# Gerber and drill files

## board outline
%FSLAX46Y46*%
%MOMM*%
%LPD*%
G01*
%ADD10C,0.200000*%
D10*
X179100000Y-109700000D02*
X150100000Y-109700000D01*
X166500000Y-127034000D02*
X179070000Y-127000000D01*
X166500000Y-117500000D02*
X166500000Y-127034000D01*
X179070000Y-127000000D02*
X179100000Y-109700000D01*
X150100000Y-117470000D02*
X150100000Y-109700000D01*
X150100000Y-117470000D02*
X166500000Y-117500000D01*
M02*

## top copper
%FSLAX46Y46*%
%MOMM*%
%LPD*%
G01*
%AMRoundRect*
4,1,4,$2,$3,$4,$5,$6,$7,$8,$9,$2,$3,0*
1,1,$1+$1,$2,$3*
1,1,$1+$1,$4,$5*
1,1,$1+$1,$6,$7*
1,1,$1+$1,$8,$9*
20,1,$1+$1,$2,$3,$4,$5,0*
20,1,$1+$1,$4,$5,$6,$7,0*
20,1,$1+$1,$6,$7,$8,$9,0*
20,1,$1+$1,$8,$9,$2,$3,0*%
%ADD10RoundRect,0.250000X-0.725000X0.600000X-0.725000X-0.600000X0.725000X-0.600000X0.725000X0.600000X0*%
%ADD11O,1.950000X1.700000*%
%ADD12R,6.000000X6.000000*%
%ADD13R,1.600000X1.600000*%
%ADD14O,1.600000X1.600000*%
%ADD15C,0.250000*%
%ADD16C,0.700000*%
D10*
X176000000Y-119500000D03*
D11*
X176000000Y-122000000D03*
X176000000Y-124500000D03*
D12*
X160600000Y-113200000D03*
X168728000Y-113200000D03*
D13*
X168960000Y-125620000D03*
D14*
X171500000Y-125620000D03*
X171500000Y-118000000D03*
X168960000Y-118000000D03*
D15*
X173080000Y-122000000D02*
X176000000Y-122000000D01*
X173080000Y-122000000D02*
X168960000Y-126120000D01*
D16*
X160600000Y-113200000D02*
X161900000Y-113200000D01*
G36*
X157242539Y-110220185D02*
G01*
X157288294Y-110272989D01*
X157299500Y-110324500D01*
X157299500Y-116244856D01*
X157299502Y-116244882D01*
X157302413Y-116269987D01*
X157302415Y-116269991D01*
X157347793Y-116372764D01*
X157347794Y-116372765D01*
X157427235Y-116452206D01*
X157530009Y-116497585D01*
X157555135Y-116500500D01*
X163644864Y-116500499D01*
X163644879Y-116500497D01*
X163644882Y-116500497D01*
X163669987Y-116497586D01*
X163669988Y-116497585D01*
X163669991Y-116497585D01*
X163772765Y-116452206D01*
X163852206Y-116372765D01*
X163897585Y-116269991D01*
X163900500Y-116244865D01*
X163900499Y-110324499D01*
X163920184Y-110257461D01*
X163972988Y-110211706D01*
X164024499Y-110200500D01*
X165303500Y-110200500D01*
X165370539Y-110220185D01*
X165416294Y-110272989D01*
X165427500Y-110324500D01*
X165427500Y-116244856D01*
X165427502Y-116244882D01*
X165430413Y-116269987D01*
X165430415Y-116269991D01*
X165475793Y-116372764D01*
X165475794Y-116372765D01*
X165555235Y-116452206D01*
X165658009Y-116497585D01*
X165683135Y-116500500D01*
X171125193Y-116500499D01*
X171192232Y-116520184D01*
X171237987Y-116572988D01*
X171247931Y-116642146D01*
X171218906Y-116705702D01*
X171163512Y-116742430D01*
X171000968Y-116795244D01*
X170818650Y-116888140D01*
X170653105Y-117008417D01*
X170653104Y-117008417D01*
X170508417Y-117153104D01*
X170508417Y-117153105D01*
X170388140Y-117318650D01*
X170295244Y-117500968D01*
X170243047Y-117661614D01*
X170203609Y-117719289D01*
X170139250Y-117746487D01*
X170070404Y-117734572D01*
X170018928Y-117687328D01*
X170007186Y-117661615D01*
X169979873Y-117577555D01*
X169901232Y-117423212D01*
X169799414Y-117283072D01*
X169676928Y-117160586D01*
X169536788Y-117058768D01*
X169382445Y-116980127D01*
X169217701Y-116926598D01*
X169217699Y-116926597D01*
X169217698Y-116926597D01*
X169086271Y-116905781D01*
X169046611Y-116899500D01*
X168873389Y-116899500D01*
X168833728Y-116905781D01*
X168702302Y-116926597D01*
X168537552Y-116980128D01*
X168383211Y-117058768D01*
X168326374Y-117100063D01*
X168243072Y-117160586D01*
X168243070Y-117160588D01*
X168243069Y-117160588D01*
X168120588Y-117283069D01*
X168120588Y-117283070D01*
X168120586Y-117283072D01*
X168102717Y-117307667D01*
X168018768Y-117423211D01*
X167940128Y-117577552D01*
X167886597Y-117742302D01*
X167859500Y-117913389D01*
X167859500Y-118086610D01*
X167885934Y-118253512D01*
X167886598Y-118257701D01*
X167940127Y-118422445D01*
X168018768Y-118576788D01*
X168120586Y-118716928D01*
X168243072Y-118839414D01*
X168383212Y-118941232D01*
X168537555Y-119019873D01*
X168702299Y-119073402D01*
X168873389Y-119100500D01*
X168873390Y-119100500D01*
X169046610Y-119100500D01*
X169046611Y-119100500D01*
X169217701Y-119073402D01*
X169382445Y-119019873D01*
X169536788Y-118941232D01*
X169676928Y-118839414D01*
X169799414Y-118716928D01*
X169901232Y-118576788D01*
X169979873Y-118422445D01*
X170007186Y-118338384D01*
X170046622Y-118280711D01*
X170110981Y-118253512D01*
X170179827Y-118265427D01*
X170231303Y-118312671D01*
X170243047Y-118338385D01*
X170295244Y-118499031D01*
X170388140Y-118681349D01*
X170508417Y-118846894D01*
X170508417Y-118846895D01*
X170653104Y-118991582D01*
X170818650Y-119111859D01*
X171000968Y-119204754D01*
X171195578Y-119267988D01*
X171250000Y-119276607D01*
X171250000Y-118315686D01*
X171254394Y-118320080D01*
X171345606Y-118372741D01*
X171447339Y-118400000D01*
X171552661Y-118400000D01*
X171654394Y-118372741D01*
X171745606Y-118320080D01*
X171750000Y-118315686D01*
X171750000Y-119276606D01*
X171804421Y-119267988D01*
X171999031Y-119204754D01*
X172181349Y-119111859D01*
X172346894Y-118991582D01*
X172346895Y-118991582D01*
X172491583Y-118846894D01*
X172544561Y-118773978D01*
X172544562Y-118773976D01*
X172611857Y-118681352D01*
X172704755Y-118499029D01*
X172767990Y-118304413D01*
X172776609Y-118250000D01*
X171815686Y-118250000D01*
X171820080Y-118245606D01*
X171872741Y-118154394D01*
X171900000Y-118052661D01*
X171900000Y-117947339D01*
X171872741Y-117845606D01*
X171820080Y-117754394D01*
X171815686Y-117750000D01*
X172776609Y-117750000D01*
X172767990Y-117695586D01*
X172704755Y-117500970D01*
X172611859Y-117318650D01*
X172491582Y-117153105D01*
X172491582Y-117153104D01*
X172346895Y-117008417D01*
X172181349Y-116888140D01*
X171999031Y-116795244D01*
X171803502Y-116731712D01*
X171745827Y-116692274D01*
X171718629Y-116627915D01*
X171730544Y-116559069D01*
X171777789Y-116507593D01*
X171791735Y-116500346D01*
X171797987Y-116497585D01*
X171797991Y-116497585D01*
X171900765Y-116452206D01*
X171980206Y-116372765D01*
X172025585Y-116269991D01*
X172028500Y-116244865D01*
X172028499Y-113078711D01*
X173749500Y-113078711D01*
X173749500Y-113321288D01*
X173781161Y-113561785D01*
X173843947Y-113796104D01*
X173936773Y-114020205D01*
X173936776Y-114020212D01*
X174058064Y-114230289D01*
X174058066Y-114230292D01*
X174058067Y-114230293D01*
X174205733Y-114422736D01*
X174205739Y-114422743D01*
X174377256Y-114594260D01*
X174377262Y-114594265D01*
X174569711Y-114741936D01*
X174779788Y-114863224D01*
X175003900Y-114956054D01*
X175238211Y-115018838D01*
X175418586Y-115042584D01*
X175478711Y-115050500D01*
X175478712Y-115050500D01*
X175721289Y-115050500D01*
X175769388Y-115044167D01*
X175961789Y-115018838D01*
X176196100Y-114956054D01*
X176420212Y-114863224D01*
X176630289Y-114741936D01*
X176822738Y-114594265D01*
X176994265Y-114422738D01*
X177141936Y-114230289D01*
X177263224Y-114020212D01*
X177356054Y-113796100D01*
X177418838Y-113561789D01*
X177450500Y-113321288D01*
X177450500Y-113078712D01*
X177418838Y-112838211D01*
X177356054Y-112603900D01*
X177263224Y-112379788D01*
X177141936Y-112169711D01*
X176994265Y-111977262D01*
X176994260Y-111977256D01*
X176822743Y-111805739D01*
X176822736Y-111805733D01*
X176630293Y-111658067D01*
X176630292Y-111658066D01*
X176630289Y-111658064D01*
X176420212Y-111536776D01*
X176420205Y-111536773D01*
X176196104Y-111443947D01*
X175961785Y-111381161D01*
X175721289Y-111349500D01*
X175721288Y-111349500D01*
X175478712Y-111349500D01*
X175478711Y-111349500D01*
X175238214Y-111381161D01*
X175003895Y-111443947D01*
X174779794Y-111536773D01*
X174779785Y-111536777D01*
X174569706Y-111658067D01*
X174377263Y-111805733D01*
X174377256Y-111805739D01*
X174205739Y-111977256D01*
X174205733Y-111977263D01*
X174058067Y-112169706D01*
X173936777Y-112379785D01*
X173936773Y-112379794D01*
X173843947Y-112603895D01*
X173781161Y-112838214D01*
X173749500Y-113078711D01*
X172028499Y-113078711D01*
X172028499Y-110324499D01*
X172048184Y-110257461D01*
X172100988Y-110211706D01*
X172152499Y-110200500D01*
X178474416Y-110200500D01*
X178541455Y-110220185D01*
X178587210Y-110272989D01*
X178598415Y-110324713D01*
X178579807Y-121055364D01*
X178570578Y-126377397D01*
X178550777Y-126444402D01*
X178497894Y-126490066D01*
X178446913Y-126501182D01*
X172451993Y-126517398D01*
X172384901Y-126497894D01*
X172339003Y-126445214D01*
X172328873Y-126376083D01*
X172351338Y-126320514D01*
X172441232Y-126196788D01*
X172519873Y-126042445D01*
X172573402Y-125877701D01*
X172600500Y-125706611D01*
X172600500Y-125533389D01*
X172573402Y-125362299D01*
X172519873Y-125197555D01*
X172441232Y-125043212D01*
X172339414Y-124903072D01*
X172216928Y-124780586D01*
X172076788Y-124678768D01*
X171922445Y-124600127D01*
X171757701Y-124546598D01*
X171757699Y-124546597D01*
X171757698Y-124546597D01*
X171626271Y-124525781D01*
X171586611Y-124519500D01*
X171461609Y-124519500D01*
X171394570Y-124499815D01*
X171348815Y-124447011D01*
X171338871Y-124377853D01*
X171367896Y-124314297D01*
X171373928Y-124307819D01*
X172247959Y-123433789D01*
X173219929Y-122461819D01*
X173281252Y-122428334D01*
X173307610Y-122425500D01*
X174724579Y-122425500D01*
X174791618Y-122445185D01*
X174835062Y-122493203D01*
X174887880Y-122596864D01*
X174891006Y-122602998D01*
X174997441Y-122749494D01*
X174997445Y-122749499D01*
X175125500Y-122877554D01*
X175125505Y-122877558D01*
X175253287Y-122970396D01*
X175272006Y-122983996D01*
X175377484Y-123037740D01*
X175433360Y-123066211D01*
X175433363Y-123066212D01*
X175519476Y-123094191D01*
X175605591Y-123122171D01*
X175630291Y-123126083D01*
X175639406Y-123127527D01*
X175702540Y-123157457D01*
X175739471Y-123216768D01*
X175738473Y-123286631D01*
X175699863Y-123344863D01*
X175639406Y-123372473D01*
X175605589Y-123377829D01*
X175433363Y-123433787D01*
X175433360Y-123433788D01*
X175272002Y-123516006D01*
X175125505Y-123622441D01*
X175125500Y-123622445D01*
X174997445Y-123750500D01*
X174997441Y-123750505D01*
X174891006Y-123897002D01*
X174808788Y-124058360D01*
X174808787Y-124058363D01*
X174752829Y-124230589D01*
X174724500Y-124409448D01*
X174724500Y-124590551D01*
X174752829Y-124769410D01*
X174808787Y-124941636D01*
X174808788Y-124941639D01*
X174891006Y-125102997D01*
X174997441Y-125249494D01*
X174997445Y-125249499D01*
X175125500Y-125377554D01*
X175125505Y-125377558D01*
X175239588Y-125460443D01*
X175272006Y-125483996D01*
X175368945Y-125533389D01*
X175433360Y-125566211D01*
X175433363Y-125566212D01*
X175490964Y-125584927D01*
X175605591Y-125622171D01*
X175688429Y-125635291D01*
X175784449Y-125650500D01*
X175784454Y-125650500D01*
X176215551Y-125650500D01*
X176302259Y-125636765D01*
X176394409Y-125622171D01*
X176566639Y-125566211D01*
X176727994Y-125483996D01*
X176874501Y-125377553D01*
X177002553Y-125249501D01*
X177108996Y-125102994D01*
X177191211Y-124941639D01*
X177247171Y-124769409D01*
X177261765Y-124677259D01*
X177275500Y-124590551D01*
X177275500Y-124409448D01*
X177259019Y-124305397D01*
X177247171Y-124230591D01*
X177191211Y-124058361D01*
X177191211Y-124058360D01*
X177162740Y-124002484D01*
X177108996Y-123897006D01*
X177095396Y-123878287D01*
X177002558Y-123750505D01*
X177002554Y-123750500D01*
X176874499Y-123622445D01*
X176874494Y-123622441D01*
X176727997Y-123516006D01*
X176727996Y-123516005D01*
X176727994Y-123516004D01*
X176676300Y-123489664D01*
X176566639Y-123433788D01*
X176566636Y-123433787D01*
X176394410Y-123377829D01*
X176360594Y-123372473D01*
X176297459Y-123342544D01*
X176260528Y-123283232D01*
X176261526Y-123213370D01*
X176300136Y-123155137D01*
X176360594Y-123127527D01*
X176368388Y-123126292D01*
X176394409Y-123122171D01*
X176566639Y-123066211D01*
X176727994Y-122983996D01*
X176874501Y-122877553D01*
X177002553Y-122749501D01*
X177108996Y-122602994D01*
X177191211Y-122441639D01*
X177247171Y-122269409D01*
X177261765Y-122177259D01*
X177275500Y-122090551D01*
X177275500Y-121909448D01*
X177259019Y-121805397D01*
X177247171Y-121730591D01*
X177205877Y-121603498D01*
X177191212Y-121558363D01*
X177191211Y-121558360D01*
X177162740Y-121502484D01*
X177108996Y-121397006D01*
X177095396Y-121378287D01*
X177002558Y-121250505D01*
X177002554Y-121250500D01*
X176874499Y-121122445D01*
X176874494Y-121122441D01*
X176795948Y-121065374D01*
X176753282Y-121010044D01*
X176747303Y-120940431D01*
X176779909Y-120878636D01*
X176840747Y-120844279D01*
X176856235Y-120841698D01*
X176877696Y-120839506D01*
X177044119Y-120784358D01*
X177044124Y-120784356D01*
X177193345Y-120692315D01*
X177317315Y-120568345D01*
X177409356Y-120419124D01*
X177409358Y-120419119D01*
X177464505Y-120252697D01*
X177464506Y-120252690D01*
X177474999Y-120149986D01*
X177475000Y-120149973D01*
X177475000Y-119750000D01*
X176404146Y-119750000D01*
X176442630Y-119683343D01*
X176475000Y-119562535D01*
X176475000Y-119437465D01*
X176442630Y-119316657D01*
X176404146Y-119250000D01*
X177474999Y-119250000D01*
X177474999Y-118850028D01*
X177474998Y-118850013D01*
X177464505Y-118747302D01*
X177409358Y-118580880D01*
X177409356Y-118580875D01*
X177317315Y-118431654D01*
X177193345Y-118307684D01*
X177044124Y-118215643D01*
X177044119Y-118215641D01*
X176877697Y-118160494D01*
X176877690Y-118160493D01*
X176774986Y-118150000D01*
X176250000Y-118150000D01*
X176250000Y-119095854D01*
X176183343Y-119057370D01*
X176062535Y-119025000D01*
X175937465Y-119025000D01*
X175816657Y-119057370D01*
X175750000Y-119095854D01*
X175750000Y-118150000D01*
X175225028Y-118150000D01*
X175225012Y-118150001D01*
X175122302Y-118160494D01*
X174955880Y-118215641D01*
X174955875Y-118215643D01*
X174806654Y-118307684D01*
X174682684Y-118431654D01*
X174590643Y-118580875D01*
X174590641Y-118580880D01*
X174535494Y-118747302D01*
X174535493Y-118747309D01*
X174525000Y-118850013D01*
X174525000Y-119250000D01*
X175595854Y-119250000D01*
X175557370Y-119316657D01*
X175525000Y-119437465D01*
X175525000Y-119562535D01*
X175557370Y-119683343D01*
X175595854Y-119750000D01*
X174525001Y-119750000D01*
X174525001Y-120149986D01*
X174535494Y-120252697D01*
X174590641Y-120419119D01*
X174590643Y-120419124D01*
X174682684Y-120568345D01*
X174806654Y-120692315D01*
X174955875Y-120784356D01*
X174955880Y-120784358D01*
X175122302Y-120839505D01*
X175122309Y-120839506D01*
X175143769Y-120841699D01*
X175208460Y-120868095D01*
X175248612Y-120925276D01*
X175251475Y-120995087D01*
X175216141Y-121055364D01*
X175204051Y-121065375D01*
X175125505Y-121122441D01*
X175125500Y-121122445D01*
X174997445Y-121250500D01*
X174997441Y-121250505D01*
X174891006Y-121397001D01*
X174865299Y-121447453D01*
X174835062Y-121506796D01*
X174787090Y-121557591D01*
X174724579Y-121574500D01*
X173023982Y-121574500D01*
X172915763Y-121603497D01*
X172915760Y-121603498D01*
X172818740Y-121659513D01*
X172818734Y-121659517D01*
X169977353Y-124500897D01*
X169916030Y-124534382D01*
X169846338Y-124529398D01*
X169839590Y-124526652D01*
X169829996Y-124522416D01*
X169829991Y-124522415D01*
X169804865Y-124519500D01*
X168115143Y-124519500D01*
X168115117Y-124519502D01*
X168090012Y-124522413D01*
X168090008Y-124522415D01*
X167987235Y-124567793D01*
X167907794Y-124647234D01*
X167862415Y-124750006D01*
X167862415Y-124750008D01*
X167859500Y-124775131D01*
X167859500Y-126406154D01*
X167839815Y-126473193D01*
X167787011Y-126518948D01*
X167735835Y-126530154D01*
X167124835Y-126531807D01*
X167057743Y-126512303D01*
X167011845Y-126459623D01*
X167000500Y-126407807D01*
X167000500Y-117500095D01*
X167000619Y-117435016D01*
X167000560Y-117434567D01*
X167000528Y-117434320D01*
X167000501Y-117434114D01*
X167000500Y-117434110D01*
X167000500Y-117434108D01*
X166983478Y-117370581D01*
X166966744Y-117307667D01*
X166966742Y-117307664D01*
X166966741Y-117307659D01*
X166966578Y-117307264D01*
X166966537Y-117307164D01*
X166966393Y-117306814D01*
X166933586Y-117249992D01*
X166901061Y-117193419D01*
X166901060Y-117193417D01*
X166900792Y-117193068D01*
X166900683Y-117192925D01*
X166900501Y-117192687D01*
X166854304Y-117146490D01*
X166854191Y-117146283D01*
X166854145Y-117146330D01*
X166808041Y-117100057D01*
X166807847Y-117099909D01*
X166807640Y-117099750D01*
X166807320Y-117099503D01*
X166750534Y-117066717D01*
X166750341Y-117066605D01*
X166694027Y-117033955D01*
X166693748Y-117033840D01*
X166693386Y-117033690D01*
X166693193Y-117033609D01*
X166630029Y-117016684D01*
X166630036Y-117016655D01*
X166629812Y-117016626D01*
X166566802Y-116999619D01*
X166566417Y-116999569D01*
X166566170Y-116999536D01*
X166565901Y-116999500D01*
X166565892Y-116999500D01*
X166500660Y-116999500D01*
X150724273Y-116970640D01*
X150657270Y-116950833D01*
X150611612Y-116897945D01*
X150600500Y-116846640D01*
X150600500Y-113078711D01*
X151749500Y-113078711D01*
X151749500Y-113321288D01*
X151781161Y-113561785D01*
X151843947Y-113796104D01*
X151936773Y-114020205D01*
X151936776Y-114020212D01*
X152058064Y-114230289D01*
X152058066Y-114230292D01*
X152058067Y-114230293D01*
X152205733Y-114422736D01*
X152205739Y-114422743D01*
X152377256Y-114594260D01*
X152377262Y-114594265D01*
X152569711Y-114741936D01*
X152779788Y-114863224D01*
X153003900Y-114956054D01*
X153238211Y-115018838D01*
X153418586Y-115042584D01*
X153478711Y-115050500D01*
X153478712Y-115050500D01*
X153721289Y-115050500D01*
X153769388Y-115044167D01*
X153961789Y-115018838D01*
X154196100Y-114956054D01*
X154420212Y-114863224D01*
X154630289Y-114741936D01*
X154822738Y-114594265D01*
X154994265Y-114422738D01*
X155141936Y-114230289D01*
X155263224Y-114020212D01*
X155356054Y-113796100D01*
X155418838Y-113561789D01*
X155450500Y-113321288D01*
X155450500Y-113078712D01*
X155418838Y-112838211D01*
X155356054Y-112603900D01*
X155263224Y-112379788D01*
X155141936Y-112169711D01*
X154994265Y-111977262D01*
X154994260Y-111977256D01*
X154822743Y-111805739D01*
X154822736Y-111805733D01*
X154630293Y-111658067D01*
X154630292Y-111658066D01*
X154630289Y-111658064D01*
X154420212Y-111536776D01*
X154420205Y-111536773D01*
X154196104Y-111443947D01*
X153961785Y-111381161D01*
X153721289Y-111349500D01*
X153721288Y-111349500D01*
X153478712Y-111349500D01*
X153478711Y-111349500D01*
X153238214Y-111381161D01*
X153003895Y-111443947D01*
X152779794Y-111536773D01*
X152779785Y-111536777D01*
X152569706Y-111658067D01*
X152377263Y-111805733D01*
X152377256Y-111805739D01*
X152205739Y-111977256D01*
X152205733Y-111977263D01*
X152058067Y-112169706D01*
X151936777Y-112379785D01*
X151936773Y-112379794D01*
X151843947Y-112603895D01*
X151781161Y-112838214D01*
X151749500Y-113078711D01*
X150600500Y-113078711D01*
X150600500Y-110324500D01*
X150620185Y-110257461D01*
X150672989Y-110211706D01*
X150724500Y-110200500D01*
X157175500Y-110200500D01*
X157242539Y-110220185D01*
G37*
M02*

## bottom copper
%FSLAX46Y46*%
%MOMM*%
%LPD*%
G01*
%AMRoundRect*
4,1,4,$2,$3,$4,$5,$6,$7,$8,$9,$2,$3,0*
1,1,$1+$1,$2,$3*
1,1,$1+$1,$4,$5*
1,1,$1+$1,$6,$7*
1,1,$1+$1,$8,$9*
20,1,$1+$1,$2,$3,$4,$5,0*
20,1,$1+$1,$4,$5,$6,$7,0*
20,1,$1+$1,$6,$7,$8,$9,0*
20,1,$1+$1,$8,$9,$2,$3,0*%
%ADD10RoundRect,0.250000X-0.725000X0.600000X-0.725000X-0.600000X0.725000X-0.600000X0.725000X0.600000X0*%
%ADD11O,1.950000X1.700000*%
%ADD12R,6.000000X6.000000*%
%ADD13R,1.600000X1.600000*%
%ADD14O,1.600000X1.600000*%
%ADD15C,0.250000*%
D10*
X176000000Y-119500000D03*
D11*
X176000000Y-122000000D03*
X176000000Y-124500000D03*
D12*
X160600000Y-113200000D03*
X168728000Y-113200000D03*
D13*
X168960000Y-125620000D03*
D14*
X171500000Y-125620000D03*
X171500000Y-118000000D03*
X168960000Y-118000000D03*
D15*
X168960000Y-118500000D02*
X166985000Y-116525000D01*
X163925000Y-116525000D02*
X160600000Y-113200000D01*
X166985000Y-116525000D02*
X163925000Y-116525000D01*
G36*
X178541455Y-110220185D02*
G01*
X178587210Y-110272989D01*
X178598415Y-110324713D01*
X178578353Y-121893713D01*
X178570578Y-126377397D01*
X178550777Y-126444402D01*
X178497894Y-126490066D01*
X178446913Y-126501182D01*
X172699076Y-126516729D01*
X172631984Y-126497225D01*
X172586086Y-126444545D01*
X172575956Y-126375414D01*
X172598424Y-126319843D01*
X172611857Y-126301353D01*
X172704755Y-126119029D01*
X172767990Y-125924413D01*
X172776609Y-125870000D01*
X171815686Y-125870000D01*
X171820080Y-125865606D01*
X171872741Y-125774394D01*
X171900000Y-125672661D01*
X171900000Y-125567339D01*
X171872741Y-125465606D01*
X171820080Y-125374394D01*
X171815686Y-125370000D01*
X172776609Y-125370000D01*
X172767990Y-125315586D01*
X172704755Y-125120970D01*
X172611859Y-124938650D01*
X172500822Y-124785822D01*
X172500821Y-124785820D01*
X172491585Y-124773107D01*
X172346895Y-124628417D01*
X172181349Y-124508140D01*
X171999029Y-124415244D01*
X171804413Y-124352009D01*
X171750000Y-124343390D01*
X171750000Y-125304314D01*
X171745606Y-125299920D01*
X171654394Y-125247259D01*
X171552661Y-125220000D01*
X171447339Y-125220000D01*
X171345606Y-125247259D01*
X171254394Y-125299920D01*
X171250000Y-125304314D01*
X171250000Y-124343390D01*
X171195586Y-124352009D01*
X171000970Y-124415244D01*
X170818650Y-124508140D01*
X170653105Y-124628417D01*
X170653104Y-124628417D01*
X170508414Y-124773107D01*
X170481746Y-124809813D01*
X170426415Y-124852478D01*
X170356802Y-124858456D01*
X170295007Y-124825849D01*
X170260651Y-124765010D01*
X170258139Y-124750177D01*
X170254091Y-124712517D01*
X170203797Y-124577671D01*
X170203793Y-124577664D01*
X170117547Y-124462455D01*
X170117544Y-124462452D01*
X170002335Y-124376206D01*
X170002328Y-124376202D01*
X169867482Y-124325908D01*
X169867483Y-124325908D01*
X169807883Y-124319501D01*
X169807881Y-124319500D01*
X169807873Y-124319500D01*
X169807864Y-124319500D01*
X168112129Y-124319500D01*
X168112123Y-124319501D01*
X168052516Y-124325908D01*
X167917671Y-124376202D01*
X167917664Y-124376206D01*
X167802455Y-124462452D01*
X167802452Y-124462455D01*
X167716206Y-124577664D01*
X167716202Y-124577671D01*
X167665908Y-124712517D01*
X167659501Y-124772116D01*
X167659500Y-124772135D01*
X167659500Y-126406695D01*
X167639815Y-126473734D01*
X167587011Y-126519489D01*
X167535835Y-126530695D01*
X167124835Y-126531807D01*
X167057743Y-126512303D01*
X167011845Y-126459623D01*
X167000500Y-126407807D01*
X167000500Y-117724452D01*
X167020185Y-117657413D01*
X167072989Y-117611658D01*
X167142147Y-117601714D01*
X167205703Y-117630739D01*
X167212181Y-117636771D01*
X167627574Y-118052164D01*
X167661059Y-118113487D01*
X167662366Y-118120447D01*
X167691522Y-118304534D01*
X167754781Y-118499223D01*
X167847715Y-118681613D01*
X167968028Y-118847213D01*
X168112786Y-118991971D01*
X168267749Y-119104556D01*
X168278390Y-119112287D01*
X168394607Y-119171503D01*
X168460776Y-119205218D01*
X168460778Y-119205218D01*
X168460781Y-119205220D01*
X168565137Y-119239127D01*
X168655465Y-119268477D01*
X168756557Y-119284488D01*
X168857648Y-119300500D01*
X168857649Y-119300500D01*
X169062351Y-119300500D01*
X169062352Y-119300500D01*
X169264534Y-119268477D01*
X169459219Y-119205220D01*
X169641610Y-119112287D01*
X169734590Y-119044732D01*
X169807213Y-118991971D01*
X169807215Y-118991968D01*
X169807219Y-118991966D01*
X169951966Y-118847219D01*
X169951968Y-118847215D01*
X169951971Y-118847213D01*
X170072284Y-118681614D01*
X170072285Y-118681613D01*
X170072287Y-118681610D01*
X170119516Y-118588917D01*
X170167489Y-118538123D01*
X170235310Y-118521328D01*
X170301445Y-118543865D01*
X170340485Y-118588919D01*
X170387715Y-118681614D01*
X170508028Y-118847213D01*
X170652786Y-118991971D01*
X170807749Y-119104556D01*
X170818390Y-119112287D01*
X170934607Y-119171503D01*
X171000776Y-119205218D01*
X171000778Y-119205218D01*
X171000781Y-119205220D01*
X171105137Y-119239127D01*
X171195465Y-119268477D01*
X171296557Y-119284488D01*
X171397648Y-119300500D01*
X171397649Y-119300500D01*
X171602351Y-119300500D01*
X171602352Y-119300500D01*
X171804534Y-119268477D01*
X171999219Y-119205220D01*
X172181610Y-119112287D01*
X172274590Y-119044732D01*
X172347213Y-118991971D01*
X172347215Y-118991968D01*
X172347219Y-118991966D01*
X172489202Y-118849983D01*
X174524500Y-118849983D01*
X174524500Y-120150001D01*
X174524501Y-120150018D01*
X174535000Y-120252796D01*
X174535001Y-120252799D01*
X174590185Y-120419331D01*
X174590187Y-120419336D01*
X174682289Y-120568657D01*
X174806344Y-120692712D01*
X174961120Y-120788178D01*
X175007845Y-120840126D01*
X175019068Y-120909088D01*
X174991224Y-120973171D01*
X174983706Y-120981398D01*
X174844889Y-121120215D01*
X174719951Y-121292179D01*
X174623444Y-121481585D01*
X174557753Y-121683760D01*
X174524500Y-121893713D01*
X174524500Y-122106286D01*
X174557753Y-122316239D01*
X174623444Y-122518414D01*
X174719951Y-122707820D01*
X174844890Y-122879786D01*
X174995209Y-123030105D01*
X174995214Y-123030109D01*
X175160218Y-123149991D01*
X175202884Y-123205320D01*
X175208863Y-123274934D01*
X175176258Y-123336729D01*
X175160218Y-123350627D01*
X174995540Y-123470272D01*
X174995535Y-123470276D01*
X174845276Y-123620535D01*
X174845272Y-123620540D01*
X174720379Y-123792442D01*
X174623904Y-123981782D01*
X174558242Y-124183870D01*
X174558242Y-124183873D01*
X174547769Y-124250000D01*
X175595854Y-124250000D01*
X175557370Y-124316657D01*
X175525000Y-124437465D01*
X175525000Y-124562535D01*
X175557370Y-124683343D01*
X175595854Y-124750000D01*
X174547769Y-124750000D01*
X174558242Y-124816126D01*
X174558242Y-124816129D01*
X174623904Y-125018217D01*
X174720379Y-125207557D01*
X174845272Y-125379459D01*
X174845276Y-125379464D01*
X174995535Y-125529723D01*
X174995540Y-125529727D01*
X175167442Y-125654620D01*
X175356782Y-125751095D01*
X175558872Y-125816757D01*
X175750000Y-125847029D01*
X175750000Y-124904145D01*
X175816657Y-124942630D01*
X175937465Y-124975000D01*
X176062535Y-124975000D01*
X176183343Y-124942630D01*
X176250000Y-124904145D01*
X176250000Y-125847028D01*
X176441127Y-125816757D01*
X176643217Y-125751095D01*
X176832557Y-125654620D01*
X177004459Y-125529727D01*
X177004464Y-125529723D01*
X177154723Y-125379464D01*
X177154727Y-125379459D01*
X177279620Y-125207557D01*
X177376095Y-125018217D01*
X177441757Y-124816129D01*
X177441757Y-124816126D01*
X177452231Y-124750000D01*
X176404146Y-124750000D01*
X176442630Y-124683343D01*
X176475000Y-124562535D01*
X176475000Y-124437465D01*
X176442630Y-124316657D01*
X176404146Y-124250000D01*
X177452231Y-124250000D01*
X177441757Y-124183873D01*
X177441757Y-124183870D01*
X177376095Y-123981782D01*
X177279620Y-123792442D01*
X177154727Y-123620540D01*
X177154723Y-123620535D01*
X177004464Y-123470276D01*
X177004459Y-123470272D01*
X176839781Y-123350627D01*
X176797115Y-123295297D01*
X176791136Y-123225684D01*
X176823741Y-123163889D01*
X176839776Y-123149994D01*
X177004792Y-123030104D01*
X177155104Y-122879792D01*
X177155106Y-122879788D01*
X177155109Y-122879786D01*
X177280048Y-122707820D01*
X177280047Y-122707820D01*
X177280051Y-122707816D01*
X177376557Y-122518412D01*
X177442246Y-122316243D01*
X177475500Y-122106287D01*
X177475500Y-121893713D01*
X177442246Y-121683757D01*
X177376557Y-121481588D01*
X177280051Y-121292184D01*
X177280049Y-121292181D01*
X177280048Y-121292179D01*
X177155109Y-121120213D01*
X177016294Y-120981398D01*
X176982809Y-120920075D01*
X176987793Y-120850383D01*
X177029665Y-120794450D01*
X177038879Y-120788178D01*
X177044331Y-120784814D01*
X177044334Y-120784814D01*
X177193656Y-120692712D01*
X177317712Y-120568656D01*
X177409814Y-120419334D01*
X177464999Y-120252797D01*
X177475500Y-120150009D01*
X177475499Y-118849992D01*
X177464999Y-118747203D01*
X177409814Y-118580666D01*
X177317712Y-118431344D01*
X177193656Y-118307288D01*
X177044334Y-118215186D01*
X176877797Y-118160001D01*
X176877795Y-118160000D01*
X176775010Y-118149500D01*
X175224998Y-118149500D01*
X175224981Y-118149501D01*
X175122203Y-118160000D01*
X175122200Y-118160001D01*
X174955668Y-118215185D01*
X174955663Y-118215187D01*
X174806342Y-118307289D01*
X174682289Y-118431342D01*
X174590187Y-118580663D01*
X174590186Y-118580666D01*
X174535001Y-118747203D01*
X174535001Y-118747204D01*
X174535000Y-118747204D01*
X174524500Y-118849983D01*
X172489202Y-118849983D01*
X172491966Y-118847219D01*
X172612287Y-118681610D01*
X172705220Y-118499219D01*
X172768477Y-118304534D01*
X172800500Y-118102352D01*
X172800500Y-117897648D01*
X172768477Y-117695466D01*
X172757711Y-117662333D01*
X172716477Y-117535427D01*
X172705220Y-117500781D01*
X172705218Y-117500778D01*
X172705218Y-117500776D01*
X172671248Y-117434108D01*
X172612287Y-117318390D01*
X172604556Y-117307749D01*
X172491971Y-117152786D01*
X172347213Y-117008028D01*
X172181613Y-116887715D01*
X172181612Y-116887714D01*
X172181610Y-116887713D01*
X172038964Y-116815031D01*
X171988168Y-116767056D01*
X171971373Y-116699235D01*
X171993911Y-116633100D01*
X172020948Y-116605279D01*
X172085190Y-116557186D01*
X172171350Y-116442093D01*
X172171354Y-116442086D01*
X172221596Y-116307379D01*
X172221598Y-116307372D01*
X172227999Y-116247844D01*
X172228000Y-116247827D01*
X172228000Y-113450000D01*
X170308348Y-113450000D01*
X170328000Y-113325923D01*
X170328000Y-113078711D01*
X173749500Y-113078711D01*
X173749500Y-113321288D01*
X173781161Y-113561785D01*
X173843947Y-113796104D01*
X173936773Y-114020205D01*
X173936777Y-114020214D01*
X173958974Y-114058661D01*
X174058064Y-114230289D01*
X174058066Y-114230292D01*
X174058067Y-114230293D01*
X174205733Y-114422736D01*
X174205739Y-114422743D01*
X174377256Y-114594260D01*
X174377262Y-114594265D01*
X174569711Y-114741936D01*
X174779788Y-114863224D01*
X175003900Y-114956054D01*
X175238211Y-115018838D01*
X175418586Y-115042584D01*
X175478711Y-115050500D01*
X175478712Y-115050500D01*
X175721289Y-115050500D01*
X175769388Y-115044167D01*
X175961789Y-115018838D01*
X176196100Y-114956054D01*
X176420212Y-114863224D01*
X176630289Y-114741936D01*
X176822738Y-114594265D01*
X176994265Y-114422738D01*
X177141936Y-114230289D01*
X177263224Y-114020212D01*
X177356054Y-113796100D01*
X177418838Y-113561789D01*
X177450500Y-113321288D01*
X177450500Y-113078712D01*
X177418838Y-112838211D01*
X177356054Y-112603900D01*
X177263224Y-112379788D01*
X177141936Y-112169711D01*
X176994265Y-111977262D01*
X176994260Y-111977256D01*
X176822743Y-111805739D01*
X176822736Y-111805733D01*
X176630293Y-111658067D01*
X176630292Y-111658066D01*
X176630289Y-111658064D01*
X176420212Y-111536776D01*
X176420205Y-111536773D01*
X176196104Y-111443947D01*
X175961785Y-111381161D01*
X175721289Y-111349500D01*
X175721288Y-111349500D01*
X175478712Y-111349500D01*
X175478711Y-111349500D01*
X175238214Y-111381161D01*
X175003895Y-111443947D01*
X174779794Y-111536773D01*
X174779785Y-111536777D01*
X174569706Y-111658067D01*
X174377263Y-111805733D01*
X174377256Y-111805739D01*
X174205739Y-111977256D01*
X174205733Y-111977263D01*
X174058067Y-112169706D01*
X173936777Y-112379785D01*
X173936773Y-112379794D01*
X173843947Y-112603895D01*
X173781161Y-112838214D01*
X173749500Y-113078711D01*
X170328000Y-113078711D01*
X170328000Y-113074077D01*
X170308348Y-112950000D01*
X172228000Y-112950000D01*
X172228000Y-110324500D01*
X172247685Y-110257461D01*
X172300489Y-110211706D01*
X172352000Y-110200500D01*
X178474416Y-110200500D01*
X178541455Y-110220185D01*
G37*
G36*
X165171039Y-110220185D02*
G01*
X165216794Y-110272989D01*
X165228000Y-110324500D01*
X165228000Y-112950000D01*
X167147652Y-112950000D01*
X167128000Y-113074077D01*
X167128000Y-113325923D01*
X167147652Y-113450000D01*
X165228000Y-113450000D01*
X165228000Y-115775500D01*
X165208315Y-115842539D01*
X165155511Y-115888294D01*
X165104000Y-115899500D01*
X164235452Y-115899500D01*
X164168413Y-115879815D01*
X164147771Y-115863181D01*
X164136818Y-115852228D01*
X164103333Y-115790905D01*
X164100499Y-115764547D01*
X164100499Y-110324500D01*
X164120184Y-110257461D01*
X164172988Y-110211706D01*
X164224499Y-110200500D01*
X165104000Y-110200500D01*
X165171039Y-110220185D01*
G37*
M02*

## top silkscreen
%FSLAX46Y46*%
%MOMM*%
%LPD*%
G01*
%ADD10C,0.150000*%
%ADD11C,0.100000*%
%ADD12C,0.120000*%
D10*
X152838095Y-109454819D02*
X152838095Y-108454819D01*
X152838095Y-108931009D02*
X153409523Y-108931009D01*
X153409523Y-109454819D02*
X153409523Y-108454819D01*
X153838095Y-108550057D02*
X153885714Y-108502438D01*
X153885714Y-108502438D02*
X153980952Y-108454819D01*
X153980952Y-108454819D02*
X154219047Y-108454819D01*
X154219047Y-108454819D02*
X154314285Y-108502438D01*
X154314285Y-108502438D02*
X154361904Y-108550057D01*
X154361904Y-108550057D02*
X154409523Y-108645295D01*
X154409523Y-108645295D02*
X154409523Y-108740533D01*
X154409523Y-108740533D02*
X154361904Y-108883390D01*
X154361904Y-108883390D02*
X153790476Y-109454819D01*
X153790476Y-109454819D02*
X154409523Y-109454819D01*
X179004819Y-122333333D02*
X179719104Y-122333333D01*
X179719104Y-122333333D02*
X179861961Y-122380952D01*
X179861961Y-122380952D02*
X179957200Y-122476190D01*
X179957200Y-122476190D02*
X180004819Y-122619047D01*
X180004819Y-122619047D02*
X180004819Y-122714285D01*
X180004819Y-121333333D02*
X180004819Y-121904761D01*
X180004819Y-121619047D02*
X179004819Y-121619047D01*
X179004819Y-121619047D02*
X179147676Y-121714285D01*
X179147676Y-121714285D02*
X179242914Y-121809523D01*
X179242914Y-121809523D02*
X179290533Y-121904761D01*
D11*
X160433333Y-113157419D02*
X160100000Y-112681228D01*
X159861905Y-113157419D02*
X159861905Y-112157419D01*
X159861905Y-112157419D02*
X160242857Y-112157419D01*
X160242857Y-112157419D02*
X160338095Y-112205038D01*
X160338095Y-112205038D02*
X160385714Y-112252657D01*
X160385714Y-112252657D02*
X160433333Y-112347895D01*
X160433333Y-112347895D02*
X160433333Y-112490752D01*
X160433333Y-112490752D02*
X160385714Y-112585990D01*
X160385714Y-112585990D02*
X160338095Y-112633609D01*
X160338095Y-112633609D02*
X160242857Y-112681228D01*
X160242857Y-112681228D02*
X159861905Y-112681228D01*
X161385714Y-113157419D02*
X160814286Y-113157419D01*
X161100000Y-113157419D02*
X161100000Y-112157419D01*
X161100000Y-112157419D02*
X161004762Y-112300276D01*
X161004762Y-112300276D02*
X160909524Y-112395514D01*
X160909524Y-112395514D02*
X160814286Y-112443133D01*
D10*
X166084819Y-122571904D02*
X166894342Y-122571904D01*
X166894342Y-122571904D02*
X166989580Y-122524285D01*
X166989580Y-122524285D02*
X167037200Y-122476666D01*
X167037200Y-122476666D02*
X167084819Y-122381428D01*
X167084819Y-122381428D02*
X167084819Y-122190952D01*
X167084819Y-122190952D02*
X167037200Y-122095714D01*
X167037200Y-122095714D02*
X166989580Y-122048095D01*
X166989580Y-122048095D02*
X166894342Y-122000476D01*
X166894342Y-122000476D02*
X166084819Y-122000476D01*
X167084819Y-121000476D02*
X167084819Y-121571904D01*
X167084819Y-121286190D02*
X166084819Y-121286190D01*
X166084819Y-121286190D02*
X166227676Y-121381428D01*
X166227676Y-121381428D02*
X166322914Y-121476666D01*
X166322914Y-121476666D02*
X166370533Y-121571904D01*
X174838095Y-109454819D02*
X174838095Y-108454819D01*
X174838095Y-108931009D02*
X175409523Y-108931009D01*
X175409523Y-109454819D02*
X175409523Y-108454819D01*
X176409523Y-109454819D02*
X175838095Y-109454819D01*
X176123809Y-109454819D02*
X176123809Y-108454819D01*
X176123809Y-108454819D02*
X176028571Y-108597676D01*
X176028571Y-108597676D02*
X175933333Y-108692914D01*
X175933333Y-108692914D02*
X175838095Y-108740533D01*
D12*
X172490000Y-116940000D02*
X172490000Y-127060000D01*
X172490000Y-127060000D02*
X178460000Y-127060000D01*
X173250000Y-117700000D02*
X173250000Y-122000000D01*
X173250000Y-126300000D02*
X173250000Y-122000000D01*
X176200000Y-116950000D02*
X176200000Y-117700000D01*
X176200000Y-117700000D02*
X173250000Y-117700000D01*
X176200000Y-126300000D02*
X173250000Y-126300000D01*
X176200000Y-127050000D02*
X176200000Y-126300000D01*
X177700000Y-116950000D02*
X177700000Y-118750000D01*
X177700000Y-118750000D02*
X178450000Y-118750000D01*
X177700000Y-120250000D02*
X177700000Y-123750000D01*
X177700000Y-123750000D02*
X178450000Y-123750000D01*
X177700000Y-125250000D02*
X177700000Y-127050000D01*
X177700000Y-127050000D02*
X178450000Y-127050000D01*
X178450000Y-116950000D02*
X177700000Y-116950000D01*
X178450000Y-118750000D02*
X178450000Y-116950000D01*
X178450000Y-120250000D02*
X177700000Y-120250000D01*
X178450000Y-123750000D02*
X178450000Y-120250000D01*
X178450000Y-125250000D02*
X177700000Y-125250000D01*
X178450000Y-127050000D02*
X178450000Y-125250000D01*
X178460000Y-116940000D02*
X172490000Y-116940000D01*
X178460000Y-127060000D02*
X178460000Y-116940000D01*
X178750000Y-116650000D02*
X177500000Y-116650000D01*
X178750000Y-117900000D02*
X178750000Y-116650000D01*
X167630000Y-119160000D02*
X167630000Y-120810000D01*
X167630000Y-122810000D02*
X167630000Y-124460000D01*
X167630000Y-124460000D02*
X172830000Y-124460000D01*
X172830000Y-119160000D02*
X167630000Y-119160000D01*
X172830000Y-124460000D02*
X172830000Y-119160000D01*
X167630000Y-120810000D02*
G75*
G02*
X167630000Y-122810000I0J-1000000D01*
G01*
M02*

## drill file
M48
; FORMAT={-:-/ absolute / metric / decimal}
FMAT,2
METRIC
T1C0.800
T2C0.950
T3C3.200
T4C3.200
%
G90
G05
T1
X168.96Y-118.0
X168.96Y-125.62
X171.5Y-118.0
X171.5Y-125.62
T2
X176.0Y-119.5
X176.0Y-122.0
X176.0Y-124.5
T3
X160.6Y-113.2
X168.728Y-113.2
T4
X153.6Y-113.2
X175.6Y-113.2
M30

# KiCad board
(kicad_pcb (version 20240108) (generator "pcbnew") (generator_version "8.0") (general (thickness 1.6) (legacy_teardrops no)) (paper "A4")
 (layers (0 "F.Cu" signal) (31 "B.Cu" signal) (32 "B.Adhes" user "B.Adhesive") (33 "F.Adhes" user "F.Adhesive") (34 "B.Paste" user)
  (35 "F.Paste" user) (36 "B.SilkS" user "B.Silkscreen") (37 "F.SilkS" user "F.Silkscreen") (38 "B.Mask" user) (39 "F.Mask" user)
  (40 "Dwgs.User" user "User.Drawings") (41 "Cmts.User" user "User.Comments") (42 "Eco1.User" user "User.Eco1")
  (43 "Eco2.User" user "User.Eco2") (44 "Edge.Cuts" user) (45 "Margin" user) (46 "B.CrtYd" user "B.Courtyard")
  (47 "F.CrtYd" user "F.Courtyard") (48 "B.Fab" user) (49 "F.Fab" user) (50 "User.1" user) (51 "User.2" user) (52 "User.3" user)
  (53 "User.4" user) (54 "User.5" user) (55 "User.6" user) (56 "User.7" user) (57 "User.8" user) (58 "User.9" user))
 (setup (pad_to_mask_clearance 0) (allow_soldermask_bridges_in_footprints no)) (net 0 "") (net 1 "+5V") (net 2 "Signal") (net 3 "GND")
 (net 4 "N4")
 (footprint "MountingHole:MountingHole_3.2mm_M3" (layer "F.Cu") (at 153.6 113.2)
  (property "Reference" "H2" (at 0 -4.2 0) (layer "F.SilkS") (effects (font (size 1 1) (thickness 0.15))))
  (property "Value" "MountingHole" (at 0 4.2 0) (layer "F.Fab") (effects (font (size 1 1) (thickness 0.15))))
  (pad "" np_thru_hole circle (at 0 0) (size 3.2 3.2) (drill 3.2) (layers "*.Cu" "*.Mask")))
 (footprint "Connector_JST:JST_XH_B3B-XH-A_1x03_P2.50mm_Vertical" (layer "F.Cu") (at 176 119.5 -90)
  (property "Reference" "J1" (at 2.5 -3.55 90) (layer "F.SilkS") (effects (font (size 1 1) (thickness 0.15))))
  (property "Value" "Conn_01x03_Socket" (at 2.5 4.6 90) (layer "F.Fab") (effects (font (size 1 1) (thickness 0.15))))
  (fp_line (start -2.56 3.51) (end 7.56 3.51) (stroke (width 0.12) (type solid)) (layer "F.SilkS"))
  (fp_line (start 7.56 3.51) (end 7.56 -2.46) (stroke (width 0.12) (type solid)) (layer "F.SilkS"))
  (fp_line (start -1.8 2.75) (end 2.5 2.75) (stroke (width 0.12) (type solid)) (layer "F.SilkS"))
  (fp_line (start 6.8 2.75) (end 2.5 2.75) (stroke (width 0.12) (type solid)) (layer "F.SilkS"))
  (fp_line (start -2.55 -0.2) (end -1.8 -0.2) (stroke (width 0.12) (type solid)) (layer "F.SilkS"))
  (fp_line (start -1.8 -0.2) (end -1.8 2.75) (stroke (width 0.12) (type solid)) (layer "F.SilkS"))
  (fp_line (start 6.8 -0.2) (end 6.8 2.75) (stroke (width 0.12) (type solid)) (layer "F.SilkS"))
  (fp_line (start 7.55 -0.2) (end 6.8 -0.2) (stroke (width 0.12) (type solid)) (layer "F.SilkS"))
  (fp_line (start -2.55 -1.7) (end -0.75 -1.7) (stroke (width 0.12) (type solid)) (layer "F.SilkS"))
  (fp_line (start -0.75 -1.7) (end -0.75 -2.45) (stroke (width 0.12) (type solid)) (layer "F.SilkS"))
  (fp_line (start 0.75 -1.7) (end 4.25 -1.7) (stroke (width 0.12) (type solid)) (layer "F.SilkS"))
  (fp_line (start 4.25 -1.7) (end 4.25 -2.45) (stroke (width 0.12) (type solid)) (layer "F.SilkS"))
  (fp_line (start 5.75 -1.7) (end 7.55 -1.7) (stroke (width 0.12) (type solid)) (layer "F.SilkS"))
  (fp_line (start 7.55 -1.7) (end 7.55 -2.45) (stroke (width 0.12) (type solid)) (layer "F.SilkS"))
  (fp_line (start -2.55 -2.45) (end -2.55 -1.7) (stroke (width 0.12) (type solid)) (layer "F.SilkS"))
  (fp_line (start -0.75 -2.45) (end -2.55 -2.45) (stroke (width 0.12) (type solid)) (layer "F.SilkS"))
  (fp_line (start 0.75 -2.45) (end 0.75 -1.7) (stroke (width 0.12) (type solid)) (layer "F.SilkS"))
  (fp_line (start 4.25 -2.45) (end 0.75 -2.45) (stroke (width 0.12) (type solid)) (layer "F.SilkS"))
  (fp_line (start 5.75 -2.45) (end 5.75 -1.7) (stroke (width 0.12) (type solid)) (layer "F.SilkS"))
  (fp_line (start 7.55 -2.45) (end 5.75 -2.45) (stroke (width 0.12) (type solid)) (layer "F.SilkS"))
  (fp_line (start -2.56 -2.46) (end -2.56 3.51) (stroke (width 0.12) (type solid)) (layer "F.SilkS"))
  (fp_line (start 7.56 -2.46) (end -2.56 -2.46) (stroke (width 0.12) (type solid)) (layer "F.SilkS"))
  (fp_line (start -2.85 -2.75) (end -2.85 -1.5) (stroke (width 0.12) (type solid)) (layer "F.SilkS"))
  (fp_line (start -1.6 -2.75) (end -2.85 -2.75) (stroke (width 0.12) (type solid)) (layer "F.SilkS"))
  (pad "1" thru_hole roundrect (at 0 0 270) (size 1.7 1.95) (drill 0.95) (layers "*.Cu" "*.Mask") (remove_unused_layers no)
   (roundrect_rratio 0.147059) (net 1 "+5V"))
  (pad "2" thru_hole oval (at 2.5 0 270) (size 1.7 1.95) (drill 0.95) (layers "*.Cu" "*.Mask") (remove_unused_layers no) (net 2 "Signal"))
  (pad "3" thru_hole oval (at 5 0 270) (size 1.7 1.95) (drill 0.95) (layers "*.Cu" "*.Mask") (remove_unused_layers no) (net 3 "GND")))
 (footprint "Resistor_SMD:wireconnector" (layer "F.Cu") (at 160.6 113.2)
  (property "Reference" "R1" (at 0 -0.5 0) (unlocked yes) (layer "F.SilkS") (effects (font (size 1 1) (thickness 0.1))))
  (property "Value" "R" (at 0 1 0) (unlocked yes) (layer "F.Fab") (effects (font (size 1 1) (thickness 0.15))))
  (pad "1" thru_hole rect (at 0 0) (size 6 6) (drill 3.2) (layers "*.Cu" "*.Mask") (remove_unused_layers no) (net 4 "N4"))
  (pad "2" thru_hole rect (at 8.128 0) (size 6 6) (drill 3.2) (layers "*.Cu" "*.Mask") (remove_unused_layers no) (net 3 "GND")))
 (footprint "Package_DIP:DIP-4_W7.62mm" (layer "F.Cu") (at 168.96 125.62 90)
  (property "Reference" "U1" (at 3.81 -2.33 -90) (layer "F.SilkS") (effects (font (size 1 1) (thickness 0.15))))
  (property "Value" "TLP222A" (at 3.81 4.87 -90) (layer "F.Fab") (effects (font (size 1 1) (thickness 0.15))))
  (fp_line (start 6.46 -1.33) (end 4.81 -1.33) (stroke (width 0.12) (type solid)) (layer "F.SilkS"))
  (fp_line (start 2.81 -1.33) (end 1.16 -1.33) (stroke (width 0.12) (type solid)) (layer "F.SilkS"))
  (fp_line (start 1.16 -1.33) (end 1.16 3.87) (stroke (width 0.12) (type solid)) (layer "F.SilkS"))
  (fp_line (start 6.46 3.87) (end 6.46 -1.33) (stroke (width 0.12) (type solid)) (layer "F.SilkS"))
  (fp_line (start 1.16 3.87) (end 6.46 3.87) (stroke (width 0.12) (type solid)) (layer "F.SilkS"))
  (fp_arc (start 4.81 -1.33) (mid 3.81 -0.33) (end 2.81 -1.33) (stroke (width 0.12) (type solid)) (layer "F.SilkS"))
  (pad "1" thru_hole rect (at 0 0 90) (size 1.6 1.6) (drill 0.8) (layers "*.Cu" "*.Mask") (remove_unused_layers no) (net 2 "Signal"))
  (pad "2" thru_hole oval (at 0 2.54 90) (size 1.6 1.6) (drill 0.8) (layers "*.Cu" "*.Mask") (remove_unused_layers no) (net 3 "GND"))
  (pad "3" thru_hole oval (at 7.62 2.54 90) (size 1.6 1.6) (drill 0.8) (layers "*.Cu" "*.Mask") (remove_unused_layers no) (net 1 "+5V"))
  (pad "4" thru_hole oval (at 7.62 0 90) (size 1.6 1.6) (drill 0.8) (layers "*.Cu" "*.Mask") (remove_unused_layers no) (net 4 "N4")))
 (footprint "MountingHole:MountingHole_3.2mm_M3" (layer "F.Cu") (at 175.6 113.2)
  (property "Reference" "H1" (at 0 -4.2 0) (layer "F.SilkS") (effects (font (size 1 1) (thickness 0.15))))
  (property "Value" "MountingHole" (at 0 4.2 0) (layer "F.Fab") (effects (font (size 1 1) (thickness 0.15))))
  (pad "" np_thru_hole circle (at 0 0) (size 3.2 3.2) (drill 3.2) (layers "*.Cu" "*.Mask")))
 (gr_line (start 179.1 109.7) (end 150.1 109.7) (stroke (width 0.2) (type default)) (layer "Edge.Cuts"))
 (gr_line (start 166.5 127.034) (end 179.07 127) (stroke (width 0.2) (type default)) (layer "Edge.Cuts"))
 (gr_line (start 166.5 117.5) (end 166.5 127.034) (stroke (width 0.2) (type default)) (layer "Edge.Cuts"))
 (gr_line (start 179.07 127) (end 179.1 109.7) (stroke (width 0.2) (type default)) (layer "Edge.Cuts"))
 (gr_line (start 150.1 117.47) (end 150.1 109.7) (stroke (width 0.2) (type default)) (layer "Edge.Cuts"))
 (gr_line (start 150.1 117.47) (end 166.5 117.5) (stroke (width 0.2) (type default)) (layer "Edge.Cuts"))
 (segment (start 173.08 122) (end 176 122) (width 0.25) (layer "F.Cu") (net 2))
 (segment (start 173.08 122) (end 168.96 126.12) (width 0.25) (layer "F.Cu") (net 2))
 (segment (start 160.6 113.2) (end 161.9 113.2) (width 0.7) (layer "F.Cu") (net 4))
 (segment (start 168.96 118.5) (end 166.985 116.525) (width 0.25) (layer "B.Cu") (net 4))
 (segment (start 163.925 116.525) (end 160.6 113.2) (width 0.25) (layer "B.Cu") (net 4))
 (segment (start 166.985 116.525) (end 163.925 116.525) (width 0.25) (layer "B.Cu") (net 4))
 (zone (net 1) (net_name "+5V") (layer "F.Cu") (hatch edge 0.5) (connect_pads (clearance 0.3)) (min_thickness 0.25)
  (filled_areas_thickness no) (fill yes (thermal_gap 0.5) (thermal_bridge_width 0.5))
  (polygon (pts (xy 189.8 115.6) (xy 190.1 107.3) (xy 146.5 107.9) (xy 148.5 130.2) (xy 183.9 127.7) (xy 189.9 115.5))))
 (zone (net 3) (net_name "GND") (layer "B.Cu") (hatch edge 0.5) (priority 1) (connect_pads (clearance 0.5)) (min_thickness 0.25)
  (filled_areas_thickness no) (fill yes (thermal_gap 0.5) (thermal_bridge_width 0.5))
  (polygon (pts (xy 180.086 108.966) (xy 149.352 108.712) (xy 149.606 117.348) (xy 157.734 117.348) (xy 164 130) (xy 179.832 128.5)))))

